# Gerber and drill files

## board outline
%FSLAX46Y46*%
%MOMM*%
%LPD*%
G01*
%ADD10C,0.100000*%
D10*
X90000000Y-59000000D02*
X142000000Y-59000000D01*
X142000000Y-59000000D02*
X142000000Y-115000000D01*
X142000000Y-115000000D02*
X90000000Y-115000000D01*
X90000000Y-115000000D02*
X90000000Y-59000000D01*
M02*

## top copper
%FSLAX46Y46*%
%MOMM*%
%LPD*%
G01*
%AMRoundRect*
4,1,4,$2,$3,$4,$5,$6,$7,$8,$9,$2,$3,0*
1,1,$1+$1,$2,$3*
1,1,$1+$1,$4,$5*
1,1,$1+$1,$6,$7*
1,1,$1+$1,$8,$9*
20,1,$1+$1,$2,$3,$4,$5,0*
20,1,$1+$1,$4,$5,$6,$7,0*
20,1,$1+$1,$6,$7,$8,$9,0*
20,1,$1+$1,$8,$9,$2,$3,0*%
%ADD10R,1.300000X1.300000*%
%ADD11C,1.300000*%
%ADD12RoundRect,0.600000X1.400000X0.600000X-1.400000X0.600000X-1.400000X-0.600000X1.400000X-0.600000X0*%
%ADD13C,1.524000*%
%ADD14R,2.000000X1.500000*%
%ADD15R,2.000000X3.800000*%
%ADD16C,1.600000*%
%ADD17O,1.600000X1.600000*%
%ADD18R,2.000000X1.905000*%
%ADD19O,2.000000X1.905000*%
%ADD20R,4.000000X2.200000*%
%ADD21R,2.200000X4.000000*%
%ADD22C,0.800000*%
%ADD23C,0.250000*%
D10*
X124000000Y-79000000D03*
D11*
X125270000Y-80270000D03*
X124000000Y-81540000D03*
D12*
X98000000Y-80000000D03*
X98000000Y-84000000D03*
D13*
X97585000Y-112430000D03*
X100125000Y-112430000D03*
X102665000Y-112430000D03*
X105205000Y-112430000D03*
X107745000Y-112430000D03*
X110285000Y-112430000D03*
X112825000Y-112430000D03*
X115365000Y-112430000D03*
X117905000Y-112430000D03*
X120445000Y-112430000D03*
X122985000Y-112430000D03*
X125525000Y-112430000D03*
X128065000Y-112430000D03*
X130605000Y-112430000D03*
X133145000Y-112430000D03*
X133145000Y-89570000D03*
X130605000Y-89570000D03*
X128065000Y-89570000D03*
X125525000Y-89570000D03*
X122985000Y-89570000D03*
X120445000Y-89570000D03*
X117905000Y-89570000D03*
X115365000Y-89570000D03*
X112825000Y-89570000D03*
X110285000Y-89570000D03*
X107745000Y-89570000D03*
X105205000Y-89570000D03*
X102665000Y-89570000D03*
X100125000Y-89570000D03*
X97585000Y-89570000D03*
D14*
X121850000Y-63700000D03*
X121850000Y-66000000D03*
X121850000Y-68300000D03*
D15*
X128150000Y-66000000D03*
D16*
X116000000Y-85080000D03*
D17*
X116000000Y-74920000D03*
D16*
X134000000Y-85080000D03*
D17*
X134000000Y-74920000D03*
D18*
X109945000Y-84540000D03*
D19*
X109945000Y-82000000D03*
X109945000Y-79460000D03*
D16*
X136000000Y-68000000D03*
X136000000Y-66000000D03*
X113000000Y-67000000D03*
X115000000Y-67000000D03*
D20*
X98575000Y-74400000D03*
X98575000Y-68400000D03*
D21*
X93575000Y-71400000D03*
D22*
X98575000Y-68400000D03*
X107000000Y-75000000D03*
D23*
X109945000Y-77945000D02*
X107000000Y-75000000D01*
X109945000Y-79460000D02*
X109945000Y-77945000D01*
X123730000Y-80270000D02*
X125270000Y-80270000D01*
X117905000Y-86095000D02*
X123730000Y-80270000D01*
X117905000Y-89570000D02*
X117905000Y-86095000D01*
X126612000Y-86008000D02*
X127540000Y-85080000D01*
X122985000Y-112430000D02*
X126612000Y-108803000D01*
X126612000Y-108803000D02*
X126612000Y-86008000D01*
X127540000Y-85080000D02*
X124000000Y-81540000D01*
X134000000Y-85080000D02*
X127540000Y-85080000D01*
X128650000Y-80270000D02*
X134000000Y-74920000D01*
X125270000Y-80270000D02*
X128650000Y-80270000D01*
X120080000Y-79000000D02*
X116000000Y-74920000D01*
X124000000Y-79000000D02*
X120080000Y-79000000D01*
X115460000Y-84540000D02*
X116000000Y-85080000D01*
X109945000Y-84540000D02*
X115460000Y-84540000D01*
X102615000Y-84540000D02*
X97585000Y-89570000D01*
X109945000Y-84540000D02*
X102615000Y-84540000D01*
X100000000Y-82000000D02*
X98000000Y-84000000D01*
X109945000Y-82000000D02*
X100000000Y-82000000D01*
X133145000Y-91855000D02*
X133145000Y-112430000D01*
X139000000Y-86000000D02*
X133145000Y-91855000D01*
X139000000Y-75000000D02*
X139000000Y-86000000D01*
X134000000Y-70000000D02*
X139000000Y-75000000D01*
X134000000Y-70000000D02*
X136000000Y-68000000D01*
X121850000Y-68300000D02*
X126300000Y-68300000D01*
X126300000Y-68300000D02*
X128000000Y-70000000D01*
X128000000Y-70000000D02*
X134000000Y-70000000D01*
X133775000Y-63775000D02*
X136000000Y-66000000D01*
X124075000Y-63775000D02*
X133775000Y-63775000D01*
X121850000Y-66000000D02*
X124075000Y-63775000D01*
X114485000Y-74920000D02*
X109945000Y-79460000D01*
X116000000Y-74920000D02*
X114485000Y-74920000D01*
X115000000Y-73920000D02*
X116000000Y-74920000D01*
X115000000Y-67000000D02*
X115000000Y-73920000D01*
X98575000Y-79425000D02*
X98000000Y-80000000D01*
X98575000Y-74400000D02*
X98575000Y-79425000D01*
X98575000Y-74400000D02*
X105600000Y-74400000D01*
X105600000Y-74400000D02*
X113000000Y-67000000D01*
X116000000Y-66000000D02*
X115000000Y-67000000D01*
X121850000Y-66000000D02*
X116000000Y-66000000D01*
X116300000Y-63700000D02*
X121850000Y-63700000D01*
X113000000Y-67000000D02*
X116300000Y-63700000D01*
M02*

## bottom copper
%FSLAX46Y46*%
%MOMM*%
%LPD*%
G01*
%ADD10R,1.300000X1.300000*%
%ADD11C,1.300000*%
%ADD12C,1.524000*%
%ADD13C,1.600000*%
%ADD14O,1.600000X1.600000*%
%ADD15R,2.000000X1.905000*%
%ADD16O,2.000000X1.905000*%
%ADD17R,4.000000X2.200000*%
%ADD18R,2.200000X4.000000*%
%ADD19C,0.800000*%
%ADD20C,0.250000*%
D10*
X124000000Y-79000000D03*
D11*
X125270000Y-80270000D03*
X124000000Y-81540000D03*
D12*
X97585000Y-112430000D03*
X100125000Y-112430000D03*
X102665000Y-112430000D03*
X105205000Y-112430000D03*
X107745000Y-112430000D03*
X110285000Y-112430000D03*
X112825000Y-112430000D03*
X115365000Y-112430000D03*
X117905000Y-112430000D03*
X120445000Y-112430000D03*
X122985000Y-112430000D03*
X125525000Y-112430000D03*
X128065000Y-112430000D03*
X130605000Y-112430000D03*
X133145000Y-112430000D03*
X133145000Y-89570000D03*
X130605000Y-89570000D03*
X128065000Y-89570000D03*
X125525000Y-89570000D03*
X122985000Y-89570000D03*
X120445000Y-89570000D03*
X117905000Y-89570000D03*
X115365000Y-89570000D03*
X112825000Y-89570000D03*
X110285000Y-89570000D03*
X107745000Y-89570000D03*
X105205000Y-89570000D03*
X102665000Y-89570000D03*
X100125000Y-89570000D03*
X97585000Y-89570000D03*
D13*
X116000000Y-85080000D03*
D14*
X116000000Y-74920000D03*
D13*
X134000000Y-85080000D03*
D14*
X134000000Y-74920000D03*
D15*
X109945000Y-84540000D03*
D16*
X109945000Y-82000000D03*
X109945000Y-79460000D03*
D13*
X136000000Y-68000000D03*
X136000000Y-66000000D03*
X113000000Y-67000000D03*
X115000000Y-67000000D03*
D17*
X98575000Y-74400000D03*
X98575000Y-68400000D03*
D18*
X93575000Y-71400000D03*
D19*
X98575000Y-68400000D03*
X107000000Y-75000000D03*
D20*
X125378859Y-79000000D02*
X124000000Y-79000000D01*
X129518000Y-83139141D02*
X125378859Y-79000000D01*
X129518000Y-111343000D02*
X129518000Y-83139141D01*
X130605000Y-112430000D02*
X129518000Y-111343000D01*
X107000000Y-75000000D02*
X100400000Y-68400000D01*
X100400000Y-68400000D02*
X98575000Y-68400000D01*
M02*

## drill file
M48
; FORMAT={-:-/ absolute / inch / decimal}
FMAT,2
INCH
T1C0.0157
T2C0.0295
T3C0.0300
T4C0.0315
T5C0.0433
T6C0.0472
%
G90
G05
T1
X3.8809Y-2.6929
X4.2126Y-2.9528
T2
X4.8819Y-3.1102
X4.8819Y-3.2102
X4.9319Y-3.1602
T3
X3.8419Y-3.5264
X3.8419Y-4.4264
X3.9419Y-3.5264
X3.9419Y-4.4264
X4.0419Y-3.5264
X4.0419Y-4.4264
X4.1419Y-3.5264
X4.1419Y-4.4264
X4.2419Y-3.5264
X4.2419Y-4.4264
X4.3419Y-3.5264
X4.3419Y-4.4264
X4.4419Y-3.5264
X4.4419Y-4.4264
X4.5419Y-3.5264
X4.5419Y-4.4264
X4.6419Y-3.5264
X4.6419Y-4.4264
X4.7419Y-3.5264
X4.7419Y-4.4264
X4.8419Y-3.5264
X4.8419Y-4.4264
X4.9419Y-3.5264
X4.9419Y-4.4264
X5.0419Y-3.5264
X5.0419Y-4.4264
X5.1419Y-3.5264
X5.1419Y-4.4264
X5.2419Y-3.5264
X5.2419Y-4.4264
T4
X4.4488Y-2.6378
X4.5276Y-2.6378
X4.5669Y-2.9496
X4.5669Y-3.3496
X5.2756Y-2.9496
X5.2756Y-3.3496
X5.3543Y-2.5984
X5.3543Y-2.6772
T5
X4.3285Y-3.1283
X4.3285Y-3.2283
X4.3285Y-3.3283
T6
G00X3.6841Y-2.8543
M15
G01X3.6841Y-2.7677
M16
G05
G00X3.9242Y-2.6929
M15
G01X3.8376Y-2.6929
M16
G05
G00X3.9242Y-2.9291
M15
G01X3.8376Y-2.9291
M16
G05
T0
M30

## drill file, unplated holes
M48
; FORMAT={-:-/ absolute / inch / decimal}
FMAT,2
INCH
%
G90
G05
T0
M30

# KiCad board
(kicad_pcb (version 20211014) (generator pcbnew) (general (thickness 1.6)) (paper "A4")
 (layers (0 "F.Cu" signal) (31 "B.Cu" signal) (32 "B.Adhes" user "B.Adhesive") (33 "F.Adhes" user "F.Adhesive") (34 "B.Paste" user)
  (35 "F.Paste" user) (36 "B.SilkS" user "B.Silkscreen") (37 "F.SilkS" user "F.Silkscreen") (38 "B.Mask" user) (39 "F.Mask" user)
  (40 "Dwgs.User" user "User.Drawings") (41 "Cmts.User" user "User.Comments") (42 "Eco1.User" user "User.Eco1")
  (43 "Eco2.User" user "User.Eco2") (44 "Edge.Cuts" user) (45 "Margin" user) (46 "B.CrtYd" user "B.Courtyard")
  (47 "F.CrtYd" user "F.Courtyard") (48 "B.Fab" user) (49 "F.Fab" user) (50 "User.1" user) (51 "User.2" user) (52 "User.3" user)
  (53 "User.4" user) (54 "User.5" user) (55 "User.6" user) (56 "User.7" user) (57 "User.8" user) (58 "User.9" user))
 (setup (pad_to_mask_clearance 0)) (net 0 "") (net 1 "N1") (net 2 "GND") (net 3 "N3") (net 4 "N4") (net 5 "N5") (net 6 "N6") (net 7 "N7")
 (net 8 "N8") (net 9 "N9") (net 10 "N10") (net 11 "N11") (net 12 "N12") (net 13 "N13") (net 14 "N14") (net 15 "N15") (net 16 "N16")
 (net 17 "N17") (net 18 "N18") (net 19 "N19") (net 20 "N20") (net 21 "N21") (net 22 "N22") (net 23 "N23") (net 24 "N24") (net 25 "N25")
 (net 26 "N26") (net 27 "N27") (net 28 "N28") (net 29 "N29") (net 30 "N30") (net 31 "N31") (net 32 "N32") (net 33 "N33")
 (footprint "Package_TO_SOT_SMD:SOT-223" (layer "F.Cu") (at 125 66)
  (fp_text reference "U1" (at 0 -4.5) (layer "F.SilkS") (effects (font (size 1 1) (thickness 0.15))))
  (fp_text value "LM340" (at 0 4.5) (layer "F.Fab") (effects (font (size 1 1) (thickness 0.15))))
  (pad "1" smd rect (at -3.15 -2.3) (size 2 1.5) (layers "F.Cu" "F.Paste" "F.Mask") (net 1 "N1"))
  (pad "2" smd rect (at -3.15 0) (size 2 1.5) (layers "F.Cu" "F.Paste" "F.Mask") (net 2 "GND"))
  (pad "3" smd rect (at -3.15 2.3) (size 2 1.5) (layers "F.Cu" "F.Paste" "F.Mask") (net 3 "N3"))
  (pad "4" smd rect (at 3.15 0) (size 2 3.8) (layers "F.Cu" "F.Paste" "F.Mask")))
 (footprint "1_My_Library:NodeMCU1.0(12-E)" (layer "F.Cu") (at 97.585 112.43 90)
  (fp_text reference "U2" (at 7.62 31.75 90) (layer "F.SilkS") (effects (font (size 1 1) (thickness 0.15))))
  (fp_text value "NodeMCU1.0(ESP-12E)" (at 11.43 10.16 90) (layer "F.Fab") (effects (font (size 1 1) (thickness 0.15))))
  (pad "1" thru_hole circle (at 0 0 90) (size 1.524 1.524) (drill 0.762) (layers *.Cu *.Mask "F.SilkS") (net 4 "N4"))
  (pad "2" thru_hole circle (at 0 2.54 90) (size 1.524 1.524) (drill 0.762) (layers *.Cu *.Mask "F.SilkS") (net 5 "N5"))
  (pad "3" thru_hole circle (at 0 5.08 90) (size 1.524 1.524) (drill 0.762) (layers *.Cu *.Mask "F.SilkS") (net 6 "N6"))
  (pad "4" thru_hole circle (at 0 7.62 90) (size 1.524 1.524) (drill 0.762) (layers *.Cu *.Mask "F.SilkS") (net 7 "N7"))
  (pad "5" thru_hole circle (at 0 10.16 90) (size 1.524 1.524) (drill 0.762) (layers *.Cu *.Mask "F.SilkS") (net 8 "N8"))
  (pad "6" thru_hole circle (at 0 12.7 90) (size 1.524 1.524) (drill 0.762) (layers *.Cu *.Mask "F.SilkS") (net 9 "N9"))
  (pad "7" thru_hole circle (at 0 15.24 90) (size 1.524 1.524) (drill 0.762) (layers *.Cu *.Mask "F.SilkS") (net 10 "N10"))
  (pad "8" thru_hole circle (at 0 17.78 90) (size 1.524 1.524) (drill 0.762) (layers *.Cu *.Mask "F.SilkS") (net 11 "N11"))
  (pad "9" thru_hole circle (at 0 20.32 90) (size 1.524 1.524) (drill 0.762) (layers *.Cu *.Mask "F.SilkS") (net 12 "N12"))
  (pad "10" thru_hole circle (at 0 22.86 90) (size 1.524 1.524) (drill 0.762) (layers *.Cu *.Mask "F.SilkS") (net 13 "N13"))
  (pad "11" thru_hole circle (at 0 25.4 90) (size 1.524 1.524) (drill 0.762) (layers *.Cu *.Mask "F.SilkS") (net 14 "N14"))
  (pad "12" thru_hole circle (at 0 27.94 90) (size 1.524 1.524) (drill 0.762) (layers *.Cu *.Mask "F.SilkS") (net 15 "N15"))
  (pad "13" thru_hole circle (at 0 30.48 90) (size 1.524 1.524) (drill 0.762) (layers *.Cu *.Mask "F.SilkS") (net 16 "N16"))
  (pad "14" thru_hole circle (at 0 33.02 90) (size 1.524 1.524) (drill 0.762) (layers *.Cu *.Mask "F.SilkS") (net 2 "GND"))
  (pad "15" thru_hole circle (at 0 35.56 90) (size 1.524 1.524) (drill 0.762) (layers *.Cu *.Mask "F.SilkS") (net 3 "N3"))
  (pad "16" thru_hole circle (at 22.86 35.56 90) (size 1.524 1.524) (drill 0.762) (layers *.Cu *.Mask "F.SilkS") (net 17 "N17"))
  (pad "17" thru_hole circle (at 22.86 33.02 90) (size 1.524 1.524) (drill 0.762) (layers *.Cu *.Mask "F.SilkS") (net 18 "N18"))
  (pad "18" thru_hole circle (at 22.86 30.48 90) (size 1.524 1.524) (drill 0.762) (layers *.Cu *.Mask "F.SilkS") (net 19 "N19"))
  (pad "19" thru_hole circle (at 22.86 27.94 90) (size 1.524 1.524) (drill 0.762) (layers *.Cu *.Mask "F.SilkS") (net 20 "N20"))
  (pad "20" thru_hole circle (at 22.86 25.4 90) (size 1.524 1.524) (drill 0.762) (layers *.Cu *.Mask "F.SilkS") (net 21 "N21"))
  (pad "21" thru_hole circle (at 22.86 22.86 90) (size 1.524 1.524) (drill 0.762) (layers *.Cu *.Mask "F.SilkS") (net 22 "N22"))
  (pad "22" thru_hole circle (at 22.86 20.32 90) (size 1.524 1.524) (drill 0.762) (layers *.Cu *.Mask "F.SilkS") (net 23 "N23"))
  (pad "23" thru_hole circle (at 22.86 17.78 90) (size 1.524 1.524) (drill 0.762) (layers *.Cu *.Mask "F.SilkS") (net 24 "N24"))
  (pad "24" thru_hole circle (at 22.86 15.24 90) (size 1.524 1.524) (drill 0.762) (layers *.Cu *.Mask "F.SilkS") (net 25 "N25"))
  (pad "25" thru_hole circle (at 22.86 12.7 90) (size 1.524 1.524) (drill 0.762) (layers *.Cu *.Mask "F.SilkS") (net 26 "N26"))
  (pad "26" thru_hole circle (at 22.86 10.16 90) (size 1.524 1.524) (drill 0.762) (layers *.Cu *.Mask "F.SilkS") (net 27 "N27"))
  (pad "27" thru_hole circle (at 22.86 7.62 90) (size 1.524 1.524) (drill 0.762) (layers *.Cu *.Mask "F.SilkS") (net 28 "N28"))
  (pad "28" thru_hole circle (at 22.86 5.08 90) (size 1.524 1.524) (drill 0.762) (layers *.Cu *.Mask "F.SilkS") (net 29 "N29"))
  (pad "29" thru_hole circle (at 22.86 2.54 90) (size 1.524 1.524) (drill 0.762) (layers *.Cu *.Mask "F.SilkS") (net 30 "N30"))
  (pad "30" thru_hole circle (at 22.86 0 90) (size 1.524 1.524) (drill 0.762) (layers *.Cu *.Mask "F.SilkS") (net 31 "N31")))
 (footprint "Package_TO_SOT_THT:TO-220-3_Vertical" (layer "F.Cu") (at 109.945 84.54 90)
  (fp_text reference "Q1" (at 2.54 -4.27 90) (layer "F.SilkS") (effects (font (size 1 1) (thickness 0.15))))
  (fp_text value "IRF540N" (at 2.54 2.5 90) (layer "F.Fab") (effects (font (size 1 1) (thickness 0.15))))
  (pad "1" thru_hole rect (at 0 0 90) (size 1.905 2) (drill 1.1) (layers *.Cu *.Mask) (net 31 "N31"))
  (pad "2" thru_hole oval (at 2.54 0 90) (size 1.905 2) (drill 1.1) (layers *.Cu *.Mask) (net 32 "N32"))
  (pad "3" thru_hole oval (at 5.08 0 90) (size 1.905 2) (drill 1.1) (layers *.Cu *.Mask) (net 2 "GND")))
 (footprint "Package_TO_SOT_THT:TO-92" (layer "F.Cu") (at 124 79 -90)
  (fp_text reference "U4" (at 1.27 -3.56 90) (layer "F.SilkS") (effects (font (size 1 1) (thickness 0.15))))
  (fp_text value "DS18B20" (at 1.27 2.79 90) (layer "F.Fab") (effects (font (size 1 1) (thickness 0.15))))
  (pad "1" thru_hole rect (at 0 0 270) (size 1.3 1.3) (drill 0.75) (layers *.Cu *.Mask) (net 2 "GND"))
  (pad "2" thru_hole circle (at 1.27 -1.27 270) (size 1.3 1.3) (drill 0.75) (layers *.Cu *.Mask) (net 23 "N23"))
  (pad "3" thru_hole circle (at 2.54 0 270) (size 1.3 1.3) (drill 0.75) (layers *.Cu *.Mask) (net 14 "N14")))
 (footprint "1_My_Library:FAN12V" (layer "F.Cu") (at 98 80 180)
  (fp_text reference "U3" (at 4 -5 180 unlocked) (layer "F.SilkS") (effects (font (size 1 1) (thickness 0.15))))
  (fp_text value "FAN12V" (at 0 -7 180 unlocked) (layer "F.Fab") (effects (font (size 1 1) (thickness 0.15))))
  (pad "1" smd roundrect (at 0 0 180) (size 4 2.4) (layers "F.Cu" "F.Paste" "F.Mask") (roundrect_rratio 0.25) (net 1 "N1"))
  (pad "2" smd roundrect (at 0 -4 180) (size 4 2.4) (layers "F.Cu" "F.Paste" "F.Mask") (roundrect_rratio 0.25) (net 32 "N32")))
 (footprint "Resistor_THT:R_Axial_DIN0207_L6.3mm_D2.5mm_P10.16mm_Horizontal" (layer "F.Cu") (at 116 85.08 90)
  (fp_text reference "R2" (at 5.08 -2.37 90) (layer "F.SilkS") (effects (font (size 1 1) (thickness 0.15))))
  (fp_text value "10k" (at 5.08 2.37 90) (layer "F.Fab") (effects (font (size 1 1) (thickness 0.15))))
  (pad "1" thru_hole circle (at 0 0 90) (size 1.6 1.6) (drill 0.8) (layers *.Cu *.Mask) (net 31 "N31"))
  (pad "2" thru_hole oval (at 10.16 0 90) (size 1.6 1.6) (drill 0.8) (layers *.Cu *.Mask) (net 2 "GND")))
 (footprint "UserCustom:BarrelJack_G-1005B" (layer "F.Cu") (at 98.575 60.6 180)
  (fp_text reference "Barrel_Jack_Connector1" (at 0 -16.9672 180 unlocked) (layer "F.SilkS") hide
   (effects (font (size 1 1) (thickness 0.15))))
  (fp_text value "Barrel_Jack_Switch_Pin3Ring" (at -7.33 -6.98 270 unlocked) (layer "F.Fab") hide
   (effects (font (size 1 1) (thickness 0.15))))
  (pad "1" thru_hole rect (at 0 -13.8 180) (size 4 2.2) (drill oval 3.4 1.2) (layers *.Cu *.Mask) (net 1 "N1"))
  (pad "2" thru_hole rect (at 0 -7.8 180) (size 4 2.2) (drill oval 3.4 1.2) (layers *.Cu *.Mask) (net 2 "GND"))
  (pad "3" thru_hole rect (at 5 -10.8 90) (size 4 2.2) (drill oval 3.4 1.2) (layers *.Cu *.Mask) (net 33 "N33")))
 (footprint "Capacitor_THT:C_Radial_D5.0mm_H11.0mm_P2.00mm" (layer "F.Cu") (at 113 67)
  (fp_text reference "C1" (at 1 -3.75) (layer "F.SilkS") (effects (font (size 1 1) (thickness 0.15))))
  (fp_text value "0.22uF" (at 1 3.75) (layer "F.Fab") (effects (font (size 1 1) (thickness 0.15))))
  (pad "1" thru_hole circle (at 0 0) (size 1.6 1.6) (drill 0.8) (layers *.Cu *.Mask) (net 1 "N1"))
  (pad "2" thru_hole circle (at 2 0) (size 1.6 1.6) (drill 0.8) (layers *.Cu *.Mask) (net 2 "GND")))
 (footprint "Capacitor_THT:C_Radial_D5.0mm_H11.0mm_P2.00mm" (layer "F.Cu") (at 136 68 90)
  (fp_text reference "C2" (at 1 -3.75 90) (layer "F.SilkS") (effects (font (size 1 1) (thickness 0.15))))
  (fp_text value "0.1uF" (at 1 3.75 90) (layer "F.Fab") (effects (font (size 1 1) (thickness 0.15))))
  (pad "1" thru_hole circle (at 0 0 90) (size 1.6 1.6) (drill 0.8) (layers *.Cu *.Mask) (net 3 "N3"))
  (pad "2" thru_hole circle (at 2 0 90) (size 1.6 1.6) (drill 0.8) (layers *.Cu *.Mask) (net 2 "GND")))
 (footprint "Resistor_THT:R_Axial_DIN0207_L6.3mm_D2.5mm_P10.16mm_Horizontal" (layer "F.Cu") (at 134 85.08 90)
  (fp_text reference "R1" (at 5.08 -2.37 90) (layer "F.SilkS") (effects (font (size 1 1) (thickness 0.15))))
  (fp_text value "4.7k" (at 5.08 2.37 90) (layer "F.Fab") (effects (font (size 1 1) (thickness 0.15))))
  (pad "1" thru_hole circle (at 0 0 90) (size 1.6 1.6) (drill 0.8) (layers *.Cu *.Mask) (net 14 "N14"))
  (pad "2" thru_hole oval (at 10.16 0 90) (size 1.6 1.6) (drill 0.8) (layers *.Cu *.Mask) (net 23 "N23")))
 (gr_rect (start 90 59) (end 142 115) (layer "Edge.Cuts") (width 0.1) (fill none))
 (segment (start 98.575 74.4) (end 105.6 74.4) (width 0.25) (layer "F.Cu") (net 1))
 (segment (start 105.6 74.4) (end 113 67) (width 0.25) (layer "F.Cu") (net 1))
 (segment (start 98.575 74.4) (end 98.575 79.425) (width 0.25) (layer "F.Cu") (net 1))
 (segment (start 116.3 63.7) (end 121.85 63.7) (width 0.25) (layer "F.Cu") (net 1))
 (segment (start 98.575 79.425) (end 98 80) (width 0.25) (layer "F.Cu") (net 1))
 (segment (start 113 67) (end 116.3 63.7) (width 0.25) (layer "F.Cu") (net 1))
 (segment (start 116 74.92) (end 114.485 74.92) (width 0.25) (layer "F.Cu") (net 2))
 (segment (start 115 67) (end 115 73.92) (width 0.25) (layer "F.Cu") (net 2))
 (segment (start 121.85 66) (end 116 66) (width 0.25) (layer "F.Cu") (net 2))
 (segment (start 133.775 63.775) (end 136 66) (width 0.25) (layer "F.Cu") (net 2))
 (segment (start 121.85 66) (end 124.075 63.775) (width 0.25) (layer "F.Cu") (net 2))
 (segment (start 120.08 79) (end 116 74.92) (width 0.25) (layer "F.Cu") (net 2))
 (segment (start 115 73.92) (end 116 74.92) (width 0.25) (layer "F.Cu") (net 2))
 (segment (start 116 66) (end 115 67) (width 0.25) (layer "F.Cu") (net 2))
 (segment (start 114.485 74.92) (end 109.945 79.46) (width 0.25) (layer "F.Cu") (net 2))
 (segment (start 109.945 79.46) (end 109.945 77.945) (width 0.25) (layer "F.Cu") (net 2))
 (segment (start 109.945 77.945) (end 107 75) (width 0.25) (layer "F.Cu") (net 2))
 (segment (start 124 79) (end 120.08 79) (width 0.25) (layer "F.Cu") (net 2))
 (segment (start 124.075 63.775) (end 133.775 63.775) (width 0.25) (layer "F.Cu") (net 2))
 (via (at 98.575 68.4) (size 0.8) (drill 0.4) (layers "F.Cu" "B.Cu") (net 2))
 (via (at 107 75) (size 0.8) (drill 0.4) (layers "F.Cu" "B.Cu") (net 2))
 (segment (start 100.4 68.4) (end 98.575 68.4) (width 0.25) (layer "B.Cu") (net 2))
 (segment (start 125.378859 79) (end 124 79) (width 0.25) (layer "B.Cu") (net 2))
 (segment (start 107 75) (end 100.4 68.4) (width 0.25) (layer "B.Cu") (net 2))
 (segment (start 129.518 83.139141) (end 125.378859 79) (width 0.25) (layer "B.Cu") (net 2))
 (segment (start 129.518 111.343) (end 129.518 83.139141) (width 0.25) (layer "B.Cu") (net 2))
 (segment (start 130.605 112.43) (end 129.518 111.343) (width 0.25) (layer "B.Cu") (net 2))
 (segment (start 128 70) (end 134 70) (width 0.25) (layer "F.Cu") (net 3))
 (segment (start 139 86) (end 133.145 91.855) (width 0.25) (layer "F.Cu") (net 3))
 (segment (start 139 75) (end 139 86) (width 0.25) (layer "F.Cu") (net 3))
 (segment (start 121.85 68.3) (end 126.3 68.3) (width 0.25) (layer "F.Cu") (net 3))
 (segment (start 134 70) (end 139 75) (width 0.25) (layer "F.Cu") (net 3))
 (segment (start 126.3 68.3) (end 128 70) (width 0.25) (layer "F.Cu") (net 3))
 (segment (start 133.145 91.855) (end 133.145 112.43) (width 0.25) (layer "F.Cu") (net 3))
 (segment (start 134 70) (end 136 68) (width 0.25) (layer "F.Cu") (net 3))
 (segment (start 115.46 84.54) (end 116 85.08) (width 0.25) (layer "F.Cu") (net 31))
 (segment (start 102.615 84.54) (end 97.585 89.57) (width 0.25) (layer "F.Cu") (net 31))
 (segment (start 109.945 84.54) (end 102.615 84.54) (width 0.25) (layer "F.Cu") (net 31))
 (segment (start 109.945 84.54) (end 115.46 84.54) (width 0.25) (layer "F.Cu") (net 31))
 (segment (start 109.945 82) (end 100 82) (width 0.25) (layer "F.Cu") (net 32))
 (segment (start 100 82) (end 98 84) (width 0.25) (layer "F.Cu") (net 32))
 (segment (start 122.985 112.43) (end 126.612 108.803) (width 0.25) (layer "F.Cu") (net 14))
 (segment (start 127.54 85.08) (end 124 81.54) (width 0.25) (layer "F.Cu") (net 14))
 (segment (start 134 85.08) (end 127.54 85.08) (width 0.25) (layer "F.Cu") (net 14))
 (segment (start 126.612 108.803) (end 126.612 86.008) (width 0.25) (layer "F.Cu") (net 14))
 (segment (start 126.612 86.008) (end 127.54 85.08) (width 0.25) (layer "F.Cu") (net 14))
 (segment (start 125.27 80.27) (end 128.65 80.27) (width 0.25) (layer "F.Cu") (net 23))
 (segment (start 117.905 86.095) (end 123.73 80.27) (width 0.25) (layer "F.Cu") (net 23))
 (segment (start 117.905 89.57) (end 117.905 86.095) (width 0.25) (layer "F.Cu") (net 23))
 (segment (start 123.73 80.27) (end 125.27 80.27) (width 0.25) (layer "F.Cu") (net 23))
 (segment (start 128.65 80.27) (end 134 74.92) (width 0.25) (layer "F.Cu") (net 23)))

